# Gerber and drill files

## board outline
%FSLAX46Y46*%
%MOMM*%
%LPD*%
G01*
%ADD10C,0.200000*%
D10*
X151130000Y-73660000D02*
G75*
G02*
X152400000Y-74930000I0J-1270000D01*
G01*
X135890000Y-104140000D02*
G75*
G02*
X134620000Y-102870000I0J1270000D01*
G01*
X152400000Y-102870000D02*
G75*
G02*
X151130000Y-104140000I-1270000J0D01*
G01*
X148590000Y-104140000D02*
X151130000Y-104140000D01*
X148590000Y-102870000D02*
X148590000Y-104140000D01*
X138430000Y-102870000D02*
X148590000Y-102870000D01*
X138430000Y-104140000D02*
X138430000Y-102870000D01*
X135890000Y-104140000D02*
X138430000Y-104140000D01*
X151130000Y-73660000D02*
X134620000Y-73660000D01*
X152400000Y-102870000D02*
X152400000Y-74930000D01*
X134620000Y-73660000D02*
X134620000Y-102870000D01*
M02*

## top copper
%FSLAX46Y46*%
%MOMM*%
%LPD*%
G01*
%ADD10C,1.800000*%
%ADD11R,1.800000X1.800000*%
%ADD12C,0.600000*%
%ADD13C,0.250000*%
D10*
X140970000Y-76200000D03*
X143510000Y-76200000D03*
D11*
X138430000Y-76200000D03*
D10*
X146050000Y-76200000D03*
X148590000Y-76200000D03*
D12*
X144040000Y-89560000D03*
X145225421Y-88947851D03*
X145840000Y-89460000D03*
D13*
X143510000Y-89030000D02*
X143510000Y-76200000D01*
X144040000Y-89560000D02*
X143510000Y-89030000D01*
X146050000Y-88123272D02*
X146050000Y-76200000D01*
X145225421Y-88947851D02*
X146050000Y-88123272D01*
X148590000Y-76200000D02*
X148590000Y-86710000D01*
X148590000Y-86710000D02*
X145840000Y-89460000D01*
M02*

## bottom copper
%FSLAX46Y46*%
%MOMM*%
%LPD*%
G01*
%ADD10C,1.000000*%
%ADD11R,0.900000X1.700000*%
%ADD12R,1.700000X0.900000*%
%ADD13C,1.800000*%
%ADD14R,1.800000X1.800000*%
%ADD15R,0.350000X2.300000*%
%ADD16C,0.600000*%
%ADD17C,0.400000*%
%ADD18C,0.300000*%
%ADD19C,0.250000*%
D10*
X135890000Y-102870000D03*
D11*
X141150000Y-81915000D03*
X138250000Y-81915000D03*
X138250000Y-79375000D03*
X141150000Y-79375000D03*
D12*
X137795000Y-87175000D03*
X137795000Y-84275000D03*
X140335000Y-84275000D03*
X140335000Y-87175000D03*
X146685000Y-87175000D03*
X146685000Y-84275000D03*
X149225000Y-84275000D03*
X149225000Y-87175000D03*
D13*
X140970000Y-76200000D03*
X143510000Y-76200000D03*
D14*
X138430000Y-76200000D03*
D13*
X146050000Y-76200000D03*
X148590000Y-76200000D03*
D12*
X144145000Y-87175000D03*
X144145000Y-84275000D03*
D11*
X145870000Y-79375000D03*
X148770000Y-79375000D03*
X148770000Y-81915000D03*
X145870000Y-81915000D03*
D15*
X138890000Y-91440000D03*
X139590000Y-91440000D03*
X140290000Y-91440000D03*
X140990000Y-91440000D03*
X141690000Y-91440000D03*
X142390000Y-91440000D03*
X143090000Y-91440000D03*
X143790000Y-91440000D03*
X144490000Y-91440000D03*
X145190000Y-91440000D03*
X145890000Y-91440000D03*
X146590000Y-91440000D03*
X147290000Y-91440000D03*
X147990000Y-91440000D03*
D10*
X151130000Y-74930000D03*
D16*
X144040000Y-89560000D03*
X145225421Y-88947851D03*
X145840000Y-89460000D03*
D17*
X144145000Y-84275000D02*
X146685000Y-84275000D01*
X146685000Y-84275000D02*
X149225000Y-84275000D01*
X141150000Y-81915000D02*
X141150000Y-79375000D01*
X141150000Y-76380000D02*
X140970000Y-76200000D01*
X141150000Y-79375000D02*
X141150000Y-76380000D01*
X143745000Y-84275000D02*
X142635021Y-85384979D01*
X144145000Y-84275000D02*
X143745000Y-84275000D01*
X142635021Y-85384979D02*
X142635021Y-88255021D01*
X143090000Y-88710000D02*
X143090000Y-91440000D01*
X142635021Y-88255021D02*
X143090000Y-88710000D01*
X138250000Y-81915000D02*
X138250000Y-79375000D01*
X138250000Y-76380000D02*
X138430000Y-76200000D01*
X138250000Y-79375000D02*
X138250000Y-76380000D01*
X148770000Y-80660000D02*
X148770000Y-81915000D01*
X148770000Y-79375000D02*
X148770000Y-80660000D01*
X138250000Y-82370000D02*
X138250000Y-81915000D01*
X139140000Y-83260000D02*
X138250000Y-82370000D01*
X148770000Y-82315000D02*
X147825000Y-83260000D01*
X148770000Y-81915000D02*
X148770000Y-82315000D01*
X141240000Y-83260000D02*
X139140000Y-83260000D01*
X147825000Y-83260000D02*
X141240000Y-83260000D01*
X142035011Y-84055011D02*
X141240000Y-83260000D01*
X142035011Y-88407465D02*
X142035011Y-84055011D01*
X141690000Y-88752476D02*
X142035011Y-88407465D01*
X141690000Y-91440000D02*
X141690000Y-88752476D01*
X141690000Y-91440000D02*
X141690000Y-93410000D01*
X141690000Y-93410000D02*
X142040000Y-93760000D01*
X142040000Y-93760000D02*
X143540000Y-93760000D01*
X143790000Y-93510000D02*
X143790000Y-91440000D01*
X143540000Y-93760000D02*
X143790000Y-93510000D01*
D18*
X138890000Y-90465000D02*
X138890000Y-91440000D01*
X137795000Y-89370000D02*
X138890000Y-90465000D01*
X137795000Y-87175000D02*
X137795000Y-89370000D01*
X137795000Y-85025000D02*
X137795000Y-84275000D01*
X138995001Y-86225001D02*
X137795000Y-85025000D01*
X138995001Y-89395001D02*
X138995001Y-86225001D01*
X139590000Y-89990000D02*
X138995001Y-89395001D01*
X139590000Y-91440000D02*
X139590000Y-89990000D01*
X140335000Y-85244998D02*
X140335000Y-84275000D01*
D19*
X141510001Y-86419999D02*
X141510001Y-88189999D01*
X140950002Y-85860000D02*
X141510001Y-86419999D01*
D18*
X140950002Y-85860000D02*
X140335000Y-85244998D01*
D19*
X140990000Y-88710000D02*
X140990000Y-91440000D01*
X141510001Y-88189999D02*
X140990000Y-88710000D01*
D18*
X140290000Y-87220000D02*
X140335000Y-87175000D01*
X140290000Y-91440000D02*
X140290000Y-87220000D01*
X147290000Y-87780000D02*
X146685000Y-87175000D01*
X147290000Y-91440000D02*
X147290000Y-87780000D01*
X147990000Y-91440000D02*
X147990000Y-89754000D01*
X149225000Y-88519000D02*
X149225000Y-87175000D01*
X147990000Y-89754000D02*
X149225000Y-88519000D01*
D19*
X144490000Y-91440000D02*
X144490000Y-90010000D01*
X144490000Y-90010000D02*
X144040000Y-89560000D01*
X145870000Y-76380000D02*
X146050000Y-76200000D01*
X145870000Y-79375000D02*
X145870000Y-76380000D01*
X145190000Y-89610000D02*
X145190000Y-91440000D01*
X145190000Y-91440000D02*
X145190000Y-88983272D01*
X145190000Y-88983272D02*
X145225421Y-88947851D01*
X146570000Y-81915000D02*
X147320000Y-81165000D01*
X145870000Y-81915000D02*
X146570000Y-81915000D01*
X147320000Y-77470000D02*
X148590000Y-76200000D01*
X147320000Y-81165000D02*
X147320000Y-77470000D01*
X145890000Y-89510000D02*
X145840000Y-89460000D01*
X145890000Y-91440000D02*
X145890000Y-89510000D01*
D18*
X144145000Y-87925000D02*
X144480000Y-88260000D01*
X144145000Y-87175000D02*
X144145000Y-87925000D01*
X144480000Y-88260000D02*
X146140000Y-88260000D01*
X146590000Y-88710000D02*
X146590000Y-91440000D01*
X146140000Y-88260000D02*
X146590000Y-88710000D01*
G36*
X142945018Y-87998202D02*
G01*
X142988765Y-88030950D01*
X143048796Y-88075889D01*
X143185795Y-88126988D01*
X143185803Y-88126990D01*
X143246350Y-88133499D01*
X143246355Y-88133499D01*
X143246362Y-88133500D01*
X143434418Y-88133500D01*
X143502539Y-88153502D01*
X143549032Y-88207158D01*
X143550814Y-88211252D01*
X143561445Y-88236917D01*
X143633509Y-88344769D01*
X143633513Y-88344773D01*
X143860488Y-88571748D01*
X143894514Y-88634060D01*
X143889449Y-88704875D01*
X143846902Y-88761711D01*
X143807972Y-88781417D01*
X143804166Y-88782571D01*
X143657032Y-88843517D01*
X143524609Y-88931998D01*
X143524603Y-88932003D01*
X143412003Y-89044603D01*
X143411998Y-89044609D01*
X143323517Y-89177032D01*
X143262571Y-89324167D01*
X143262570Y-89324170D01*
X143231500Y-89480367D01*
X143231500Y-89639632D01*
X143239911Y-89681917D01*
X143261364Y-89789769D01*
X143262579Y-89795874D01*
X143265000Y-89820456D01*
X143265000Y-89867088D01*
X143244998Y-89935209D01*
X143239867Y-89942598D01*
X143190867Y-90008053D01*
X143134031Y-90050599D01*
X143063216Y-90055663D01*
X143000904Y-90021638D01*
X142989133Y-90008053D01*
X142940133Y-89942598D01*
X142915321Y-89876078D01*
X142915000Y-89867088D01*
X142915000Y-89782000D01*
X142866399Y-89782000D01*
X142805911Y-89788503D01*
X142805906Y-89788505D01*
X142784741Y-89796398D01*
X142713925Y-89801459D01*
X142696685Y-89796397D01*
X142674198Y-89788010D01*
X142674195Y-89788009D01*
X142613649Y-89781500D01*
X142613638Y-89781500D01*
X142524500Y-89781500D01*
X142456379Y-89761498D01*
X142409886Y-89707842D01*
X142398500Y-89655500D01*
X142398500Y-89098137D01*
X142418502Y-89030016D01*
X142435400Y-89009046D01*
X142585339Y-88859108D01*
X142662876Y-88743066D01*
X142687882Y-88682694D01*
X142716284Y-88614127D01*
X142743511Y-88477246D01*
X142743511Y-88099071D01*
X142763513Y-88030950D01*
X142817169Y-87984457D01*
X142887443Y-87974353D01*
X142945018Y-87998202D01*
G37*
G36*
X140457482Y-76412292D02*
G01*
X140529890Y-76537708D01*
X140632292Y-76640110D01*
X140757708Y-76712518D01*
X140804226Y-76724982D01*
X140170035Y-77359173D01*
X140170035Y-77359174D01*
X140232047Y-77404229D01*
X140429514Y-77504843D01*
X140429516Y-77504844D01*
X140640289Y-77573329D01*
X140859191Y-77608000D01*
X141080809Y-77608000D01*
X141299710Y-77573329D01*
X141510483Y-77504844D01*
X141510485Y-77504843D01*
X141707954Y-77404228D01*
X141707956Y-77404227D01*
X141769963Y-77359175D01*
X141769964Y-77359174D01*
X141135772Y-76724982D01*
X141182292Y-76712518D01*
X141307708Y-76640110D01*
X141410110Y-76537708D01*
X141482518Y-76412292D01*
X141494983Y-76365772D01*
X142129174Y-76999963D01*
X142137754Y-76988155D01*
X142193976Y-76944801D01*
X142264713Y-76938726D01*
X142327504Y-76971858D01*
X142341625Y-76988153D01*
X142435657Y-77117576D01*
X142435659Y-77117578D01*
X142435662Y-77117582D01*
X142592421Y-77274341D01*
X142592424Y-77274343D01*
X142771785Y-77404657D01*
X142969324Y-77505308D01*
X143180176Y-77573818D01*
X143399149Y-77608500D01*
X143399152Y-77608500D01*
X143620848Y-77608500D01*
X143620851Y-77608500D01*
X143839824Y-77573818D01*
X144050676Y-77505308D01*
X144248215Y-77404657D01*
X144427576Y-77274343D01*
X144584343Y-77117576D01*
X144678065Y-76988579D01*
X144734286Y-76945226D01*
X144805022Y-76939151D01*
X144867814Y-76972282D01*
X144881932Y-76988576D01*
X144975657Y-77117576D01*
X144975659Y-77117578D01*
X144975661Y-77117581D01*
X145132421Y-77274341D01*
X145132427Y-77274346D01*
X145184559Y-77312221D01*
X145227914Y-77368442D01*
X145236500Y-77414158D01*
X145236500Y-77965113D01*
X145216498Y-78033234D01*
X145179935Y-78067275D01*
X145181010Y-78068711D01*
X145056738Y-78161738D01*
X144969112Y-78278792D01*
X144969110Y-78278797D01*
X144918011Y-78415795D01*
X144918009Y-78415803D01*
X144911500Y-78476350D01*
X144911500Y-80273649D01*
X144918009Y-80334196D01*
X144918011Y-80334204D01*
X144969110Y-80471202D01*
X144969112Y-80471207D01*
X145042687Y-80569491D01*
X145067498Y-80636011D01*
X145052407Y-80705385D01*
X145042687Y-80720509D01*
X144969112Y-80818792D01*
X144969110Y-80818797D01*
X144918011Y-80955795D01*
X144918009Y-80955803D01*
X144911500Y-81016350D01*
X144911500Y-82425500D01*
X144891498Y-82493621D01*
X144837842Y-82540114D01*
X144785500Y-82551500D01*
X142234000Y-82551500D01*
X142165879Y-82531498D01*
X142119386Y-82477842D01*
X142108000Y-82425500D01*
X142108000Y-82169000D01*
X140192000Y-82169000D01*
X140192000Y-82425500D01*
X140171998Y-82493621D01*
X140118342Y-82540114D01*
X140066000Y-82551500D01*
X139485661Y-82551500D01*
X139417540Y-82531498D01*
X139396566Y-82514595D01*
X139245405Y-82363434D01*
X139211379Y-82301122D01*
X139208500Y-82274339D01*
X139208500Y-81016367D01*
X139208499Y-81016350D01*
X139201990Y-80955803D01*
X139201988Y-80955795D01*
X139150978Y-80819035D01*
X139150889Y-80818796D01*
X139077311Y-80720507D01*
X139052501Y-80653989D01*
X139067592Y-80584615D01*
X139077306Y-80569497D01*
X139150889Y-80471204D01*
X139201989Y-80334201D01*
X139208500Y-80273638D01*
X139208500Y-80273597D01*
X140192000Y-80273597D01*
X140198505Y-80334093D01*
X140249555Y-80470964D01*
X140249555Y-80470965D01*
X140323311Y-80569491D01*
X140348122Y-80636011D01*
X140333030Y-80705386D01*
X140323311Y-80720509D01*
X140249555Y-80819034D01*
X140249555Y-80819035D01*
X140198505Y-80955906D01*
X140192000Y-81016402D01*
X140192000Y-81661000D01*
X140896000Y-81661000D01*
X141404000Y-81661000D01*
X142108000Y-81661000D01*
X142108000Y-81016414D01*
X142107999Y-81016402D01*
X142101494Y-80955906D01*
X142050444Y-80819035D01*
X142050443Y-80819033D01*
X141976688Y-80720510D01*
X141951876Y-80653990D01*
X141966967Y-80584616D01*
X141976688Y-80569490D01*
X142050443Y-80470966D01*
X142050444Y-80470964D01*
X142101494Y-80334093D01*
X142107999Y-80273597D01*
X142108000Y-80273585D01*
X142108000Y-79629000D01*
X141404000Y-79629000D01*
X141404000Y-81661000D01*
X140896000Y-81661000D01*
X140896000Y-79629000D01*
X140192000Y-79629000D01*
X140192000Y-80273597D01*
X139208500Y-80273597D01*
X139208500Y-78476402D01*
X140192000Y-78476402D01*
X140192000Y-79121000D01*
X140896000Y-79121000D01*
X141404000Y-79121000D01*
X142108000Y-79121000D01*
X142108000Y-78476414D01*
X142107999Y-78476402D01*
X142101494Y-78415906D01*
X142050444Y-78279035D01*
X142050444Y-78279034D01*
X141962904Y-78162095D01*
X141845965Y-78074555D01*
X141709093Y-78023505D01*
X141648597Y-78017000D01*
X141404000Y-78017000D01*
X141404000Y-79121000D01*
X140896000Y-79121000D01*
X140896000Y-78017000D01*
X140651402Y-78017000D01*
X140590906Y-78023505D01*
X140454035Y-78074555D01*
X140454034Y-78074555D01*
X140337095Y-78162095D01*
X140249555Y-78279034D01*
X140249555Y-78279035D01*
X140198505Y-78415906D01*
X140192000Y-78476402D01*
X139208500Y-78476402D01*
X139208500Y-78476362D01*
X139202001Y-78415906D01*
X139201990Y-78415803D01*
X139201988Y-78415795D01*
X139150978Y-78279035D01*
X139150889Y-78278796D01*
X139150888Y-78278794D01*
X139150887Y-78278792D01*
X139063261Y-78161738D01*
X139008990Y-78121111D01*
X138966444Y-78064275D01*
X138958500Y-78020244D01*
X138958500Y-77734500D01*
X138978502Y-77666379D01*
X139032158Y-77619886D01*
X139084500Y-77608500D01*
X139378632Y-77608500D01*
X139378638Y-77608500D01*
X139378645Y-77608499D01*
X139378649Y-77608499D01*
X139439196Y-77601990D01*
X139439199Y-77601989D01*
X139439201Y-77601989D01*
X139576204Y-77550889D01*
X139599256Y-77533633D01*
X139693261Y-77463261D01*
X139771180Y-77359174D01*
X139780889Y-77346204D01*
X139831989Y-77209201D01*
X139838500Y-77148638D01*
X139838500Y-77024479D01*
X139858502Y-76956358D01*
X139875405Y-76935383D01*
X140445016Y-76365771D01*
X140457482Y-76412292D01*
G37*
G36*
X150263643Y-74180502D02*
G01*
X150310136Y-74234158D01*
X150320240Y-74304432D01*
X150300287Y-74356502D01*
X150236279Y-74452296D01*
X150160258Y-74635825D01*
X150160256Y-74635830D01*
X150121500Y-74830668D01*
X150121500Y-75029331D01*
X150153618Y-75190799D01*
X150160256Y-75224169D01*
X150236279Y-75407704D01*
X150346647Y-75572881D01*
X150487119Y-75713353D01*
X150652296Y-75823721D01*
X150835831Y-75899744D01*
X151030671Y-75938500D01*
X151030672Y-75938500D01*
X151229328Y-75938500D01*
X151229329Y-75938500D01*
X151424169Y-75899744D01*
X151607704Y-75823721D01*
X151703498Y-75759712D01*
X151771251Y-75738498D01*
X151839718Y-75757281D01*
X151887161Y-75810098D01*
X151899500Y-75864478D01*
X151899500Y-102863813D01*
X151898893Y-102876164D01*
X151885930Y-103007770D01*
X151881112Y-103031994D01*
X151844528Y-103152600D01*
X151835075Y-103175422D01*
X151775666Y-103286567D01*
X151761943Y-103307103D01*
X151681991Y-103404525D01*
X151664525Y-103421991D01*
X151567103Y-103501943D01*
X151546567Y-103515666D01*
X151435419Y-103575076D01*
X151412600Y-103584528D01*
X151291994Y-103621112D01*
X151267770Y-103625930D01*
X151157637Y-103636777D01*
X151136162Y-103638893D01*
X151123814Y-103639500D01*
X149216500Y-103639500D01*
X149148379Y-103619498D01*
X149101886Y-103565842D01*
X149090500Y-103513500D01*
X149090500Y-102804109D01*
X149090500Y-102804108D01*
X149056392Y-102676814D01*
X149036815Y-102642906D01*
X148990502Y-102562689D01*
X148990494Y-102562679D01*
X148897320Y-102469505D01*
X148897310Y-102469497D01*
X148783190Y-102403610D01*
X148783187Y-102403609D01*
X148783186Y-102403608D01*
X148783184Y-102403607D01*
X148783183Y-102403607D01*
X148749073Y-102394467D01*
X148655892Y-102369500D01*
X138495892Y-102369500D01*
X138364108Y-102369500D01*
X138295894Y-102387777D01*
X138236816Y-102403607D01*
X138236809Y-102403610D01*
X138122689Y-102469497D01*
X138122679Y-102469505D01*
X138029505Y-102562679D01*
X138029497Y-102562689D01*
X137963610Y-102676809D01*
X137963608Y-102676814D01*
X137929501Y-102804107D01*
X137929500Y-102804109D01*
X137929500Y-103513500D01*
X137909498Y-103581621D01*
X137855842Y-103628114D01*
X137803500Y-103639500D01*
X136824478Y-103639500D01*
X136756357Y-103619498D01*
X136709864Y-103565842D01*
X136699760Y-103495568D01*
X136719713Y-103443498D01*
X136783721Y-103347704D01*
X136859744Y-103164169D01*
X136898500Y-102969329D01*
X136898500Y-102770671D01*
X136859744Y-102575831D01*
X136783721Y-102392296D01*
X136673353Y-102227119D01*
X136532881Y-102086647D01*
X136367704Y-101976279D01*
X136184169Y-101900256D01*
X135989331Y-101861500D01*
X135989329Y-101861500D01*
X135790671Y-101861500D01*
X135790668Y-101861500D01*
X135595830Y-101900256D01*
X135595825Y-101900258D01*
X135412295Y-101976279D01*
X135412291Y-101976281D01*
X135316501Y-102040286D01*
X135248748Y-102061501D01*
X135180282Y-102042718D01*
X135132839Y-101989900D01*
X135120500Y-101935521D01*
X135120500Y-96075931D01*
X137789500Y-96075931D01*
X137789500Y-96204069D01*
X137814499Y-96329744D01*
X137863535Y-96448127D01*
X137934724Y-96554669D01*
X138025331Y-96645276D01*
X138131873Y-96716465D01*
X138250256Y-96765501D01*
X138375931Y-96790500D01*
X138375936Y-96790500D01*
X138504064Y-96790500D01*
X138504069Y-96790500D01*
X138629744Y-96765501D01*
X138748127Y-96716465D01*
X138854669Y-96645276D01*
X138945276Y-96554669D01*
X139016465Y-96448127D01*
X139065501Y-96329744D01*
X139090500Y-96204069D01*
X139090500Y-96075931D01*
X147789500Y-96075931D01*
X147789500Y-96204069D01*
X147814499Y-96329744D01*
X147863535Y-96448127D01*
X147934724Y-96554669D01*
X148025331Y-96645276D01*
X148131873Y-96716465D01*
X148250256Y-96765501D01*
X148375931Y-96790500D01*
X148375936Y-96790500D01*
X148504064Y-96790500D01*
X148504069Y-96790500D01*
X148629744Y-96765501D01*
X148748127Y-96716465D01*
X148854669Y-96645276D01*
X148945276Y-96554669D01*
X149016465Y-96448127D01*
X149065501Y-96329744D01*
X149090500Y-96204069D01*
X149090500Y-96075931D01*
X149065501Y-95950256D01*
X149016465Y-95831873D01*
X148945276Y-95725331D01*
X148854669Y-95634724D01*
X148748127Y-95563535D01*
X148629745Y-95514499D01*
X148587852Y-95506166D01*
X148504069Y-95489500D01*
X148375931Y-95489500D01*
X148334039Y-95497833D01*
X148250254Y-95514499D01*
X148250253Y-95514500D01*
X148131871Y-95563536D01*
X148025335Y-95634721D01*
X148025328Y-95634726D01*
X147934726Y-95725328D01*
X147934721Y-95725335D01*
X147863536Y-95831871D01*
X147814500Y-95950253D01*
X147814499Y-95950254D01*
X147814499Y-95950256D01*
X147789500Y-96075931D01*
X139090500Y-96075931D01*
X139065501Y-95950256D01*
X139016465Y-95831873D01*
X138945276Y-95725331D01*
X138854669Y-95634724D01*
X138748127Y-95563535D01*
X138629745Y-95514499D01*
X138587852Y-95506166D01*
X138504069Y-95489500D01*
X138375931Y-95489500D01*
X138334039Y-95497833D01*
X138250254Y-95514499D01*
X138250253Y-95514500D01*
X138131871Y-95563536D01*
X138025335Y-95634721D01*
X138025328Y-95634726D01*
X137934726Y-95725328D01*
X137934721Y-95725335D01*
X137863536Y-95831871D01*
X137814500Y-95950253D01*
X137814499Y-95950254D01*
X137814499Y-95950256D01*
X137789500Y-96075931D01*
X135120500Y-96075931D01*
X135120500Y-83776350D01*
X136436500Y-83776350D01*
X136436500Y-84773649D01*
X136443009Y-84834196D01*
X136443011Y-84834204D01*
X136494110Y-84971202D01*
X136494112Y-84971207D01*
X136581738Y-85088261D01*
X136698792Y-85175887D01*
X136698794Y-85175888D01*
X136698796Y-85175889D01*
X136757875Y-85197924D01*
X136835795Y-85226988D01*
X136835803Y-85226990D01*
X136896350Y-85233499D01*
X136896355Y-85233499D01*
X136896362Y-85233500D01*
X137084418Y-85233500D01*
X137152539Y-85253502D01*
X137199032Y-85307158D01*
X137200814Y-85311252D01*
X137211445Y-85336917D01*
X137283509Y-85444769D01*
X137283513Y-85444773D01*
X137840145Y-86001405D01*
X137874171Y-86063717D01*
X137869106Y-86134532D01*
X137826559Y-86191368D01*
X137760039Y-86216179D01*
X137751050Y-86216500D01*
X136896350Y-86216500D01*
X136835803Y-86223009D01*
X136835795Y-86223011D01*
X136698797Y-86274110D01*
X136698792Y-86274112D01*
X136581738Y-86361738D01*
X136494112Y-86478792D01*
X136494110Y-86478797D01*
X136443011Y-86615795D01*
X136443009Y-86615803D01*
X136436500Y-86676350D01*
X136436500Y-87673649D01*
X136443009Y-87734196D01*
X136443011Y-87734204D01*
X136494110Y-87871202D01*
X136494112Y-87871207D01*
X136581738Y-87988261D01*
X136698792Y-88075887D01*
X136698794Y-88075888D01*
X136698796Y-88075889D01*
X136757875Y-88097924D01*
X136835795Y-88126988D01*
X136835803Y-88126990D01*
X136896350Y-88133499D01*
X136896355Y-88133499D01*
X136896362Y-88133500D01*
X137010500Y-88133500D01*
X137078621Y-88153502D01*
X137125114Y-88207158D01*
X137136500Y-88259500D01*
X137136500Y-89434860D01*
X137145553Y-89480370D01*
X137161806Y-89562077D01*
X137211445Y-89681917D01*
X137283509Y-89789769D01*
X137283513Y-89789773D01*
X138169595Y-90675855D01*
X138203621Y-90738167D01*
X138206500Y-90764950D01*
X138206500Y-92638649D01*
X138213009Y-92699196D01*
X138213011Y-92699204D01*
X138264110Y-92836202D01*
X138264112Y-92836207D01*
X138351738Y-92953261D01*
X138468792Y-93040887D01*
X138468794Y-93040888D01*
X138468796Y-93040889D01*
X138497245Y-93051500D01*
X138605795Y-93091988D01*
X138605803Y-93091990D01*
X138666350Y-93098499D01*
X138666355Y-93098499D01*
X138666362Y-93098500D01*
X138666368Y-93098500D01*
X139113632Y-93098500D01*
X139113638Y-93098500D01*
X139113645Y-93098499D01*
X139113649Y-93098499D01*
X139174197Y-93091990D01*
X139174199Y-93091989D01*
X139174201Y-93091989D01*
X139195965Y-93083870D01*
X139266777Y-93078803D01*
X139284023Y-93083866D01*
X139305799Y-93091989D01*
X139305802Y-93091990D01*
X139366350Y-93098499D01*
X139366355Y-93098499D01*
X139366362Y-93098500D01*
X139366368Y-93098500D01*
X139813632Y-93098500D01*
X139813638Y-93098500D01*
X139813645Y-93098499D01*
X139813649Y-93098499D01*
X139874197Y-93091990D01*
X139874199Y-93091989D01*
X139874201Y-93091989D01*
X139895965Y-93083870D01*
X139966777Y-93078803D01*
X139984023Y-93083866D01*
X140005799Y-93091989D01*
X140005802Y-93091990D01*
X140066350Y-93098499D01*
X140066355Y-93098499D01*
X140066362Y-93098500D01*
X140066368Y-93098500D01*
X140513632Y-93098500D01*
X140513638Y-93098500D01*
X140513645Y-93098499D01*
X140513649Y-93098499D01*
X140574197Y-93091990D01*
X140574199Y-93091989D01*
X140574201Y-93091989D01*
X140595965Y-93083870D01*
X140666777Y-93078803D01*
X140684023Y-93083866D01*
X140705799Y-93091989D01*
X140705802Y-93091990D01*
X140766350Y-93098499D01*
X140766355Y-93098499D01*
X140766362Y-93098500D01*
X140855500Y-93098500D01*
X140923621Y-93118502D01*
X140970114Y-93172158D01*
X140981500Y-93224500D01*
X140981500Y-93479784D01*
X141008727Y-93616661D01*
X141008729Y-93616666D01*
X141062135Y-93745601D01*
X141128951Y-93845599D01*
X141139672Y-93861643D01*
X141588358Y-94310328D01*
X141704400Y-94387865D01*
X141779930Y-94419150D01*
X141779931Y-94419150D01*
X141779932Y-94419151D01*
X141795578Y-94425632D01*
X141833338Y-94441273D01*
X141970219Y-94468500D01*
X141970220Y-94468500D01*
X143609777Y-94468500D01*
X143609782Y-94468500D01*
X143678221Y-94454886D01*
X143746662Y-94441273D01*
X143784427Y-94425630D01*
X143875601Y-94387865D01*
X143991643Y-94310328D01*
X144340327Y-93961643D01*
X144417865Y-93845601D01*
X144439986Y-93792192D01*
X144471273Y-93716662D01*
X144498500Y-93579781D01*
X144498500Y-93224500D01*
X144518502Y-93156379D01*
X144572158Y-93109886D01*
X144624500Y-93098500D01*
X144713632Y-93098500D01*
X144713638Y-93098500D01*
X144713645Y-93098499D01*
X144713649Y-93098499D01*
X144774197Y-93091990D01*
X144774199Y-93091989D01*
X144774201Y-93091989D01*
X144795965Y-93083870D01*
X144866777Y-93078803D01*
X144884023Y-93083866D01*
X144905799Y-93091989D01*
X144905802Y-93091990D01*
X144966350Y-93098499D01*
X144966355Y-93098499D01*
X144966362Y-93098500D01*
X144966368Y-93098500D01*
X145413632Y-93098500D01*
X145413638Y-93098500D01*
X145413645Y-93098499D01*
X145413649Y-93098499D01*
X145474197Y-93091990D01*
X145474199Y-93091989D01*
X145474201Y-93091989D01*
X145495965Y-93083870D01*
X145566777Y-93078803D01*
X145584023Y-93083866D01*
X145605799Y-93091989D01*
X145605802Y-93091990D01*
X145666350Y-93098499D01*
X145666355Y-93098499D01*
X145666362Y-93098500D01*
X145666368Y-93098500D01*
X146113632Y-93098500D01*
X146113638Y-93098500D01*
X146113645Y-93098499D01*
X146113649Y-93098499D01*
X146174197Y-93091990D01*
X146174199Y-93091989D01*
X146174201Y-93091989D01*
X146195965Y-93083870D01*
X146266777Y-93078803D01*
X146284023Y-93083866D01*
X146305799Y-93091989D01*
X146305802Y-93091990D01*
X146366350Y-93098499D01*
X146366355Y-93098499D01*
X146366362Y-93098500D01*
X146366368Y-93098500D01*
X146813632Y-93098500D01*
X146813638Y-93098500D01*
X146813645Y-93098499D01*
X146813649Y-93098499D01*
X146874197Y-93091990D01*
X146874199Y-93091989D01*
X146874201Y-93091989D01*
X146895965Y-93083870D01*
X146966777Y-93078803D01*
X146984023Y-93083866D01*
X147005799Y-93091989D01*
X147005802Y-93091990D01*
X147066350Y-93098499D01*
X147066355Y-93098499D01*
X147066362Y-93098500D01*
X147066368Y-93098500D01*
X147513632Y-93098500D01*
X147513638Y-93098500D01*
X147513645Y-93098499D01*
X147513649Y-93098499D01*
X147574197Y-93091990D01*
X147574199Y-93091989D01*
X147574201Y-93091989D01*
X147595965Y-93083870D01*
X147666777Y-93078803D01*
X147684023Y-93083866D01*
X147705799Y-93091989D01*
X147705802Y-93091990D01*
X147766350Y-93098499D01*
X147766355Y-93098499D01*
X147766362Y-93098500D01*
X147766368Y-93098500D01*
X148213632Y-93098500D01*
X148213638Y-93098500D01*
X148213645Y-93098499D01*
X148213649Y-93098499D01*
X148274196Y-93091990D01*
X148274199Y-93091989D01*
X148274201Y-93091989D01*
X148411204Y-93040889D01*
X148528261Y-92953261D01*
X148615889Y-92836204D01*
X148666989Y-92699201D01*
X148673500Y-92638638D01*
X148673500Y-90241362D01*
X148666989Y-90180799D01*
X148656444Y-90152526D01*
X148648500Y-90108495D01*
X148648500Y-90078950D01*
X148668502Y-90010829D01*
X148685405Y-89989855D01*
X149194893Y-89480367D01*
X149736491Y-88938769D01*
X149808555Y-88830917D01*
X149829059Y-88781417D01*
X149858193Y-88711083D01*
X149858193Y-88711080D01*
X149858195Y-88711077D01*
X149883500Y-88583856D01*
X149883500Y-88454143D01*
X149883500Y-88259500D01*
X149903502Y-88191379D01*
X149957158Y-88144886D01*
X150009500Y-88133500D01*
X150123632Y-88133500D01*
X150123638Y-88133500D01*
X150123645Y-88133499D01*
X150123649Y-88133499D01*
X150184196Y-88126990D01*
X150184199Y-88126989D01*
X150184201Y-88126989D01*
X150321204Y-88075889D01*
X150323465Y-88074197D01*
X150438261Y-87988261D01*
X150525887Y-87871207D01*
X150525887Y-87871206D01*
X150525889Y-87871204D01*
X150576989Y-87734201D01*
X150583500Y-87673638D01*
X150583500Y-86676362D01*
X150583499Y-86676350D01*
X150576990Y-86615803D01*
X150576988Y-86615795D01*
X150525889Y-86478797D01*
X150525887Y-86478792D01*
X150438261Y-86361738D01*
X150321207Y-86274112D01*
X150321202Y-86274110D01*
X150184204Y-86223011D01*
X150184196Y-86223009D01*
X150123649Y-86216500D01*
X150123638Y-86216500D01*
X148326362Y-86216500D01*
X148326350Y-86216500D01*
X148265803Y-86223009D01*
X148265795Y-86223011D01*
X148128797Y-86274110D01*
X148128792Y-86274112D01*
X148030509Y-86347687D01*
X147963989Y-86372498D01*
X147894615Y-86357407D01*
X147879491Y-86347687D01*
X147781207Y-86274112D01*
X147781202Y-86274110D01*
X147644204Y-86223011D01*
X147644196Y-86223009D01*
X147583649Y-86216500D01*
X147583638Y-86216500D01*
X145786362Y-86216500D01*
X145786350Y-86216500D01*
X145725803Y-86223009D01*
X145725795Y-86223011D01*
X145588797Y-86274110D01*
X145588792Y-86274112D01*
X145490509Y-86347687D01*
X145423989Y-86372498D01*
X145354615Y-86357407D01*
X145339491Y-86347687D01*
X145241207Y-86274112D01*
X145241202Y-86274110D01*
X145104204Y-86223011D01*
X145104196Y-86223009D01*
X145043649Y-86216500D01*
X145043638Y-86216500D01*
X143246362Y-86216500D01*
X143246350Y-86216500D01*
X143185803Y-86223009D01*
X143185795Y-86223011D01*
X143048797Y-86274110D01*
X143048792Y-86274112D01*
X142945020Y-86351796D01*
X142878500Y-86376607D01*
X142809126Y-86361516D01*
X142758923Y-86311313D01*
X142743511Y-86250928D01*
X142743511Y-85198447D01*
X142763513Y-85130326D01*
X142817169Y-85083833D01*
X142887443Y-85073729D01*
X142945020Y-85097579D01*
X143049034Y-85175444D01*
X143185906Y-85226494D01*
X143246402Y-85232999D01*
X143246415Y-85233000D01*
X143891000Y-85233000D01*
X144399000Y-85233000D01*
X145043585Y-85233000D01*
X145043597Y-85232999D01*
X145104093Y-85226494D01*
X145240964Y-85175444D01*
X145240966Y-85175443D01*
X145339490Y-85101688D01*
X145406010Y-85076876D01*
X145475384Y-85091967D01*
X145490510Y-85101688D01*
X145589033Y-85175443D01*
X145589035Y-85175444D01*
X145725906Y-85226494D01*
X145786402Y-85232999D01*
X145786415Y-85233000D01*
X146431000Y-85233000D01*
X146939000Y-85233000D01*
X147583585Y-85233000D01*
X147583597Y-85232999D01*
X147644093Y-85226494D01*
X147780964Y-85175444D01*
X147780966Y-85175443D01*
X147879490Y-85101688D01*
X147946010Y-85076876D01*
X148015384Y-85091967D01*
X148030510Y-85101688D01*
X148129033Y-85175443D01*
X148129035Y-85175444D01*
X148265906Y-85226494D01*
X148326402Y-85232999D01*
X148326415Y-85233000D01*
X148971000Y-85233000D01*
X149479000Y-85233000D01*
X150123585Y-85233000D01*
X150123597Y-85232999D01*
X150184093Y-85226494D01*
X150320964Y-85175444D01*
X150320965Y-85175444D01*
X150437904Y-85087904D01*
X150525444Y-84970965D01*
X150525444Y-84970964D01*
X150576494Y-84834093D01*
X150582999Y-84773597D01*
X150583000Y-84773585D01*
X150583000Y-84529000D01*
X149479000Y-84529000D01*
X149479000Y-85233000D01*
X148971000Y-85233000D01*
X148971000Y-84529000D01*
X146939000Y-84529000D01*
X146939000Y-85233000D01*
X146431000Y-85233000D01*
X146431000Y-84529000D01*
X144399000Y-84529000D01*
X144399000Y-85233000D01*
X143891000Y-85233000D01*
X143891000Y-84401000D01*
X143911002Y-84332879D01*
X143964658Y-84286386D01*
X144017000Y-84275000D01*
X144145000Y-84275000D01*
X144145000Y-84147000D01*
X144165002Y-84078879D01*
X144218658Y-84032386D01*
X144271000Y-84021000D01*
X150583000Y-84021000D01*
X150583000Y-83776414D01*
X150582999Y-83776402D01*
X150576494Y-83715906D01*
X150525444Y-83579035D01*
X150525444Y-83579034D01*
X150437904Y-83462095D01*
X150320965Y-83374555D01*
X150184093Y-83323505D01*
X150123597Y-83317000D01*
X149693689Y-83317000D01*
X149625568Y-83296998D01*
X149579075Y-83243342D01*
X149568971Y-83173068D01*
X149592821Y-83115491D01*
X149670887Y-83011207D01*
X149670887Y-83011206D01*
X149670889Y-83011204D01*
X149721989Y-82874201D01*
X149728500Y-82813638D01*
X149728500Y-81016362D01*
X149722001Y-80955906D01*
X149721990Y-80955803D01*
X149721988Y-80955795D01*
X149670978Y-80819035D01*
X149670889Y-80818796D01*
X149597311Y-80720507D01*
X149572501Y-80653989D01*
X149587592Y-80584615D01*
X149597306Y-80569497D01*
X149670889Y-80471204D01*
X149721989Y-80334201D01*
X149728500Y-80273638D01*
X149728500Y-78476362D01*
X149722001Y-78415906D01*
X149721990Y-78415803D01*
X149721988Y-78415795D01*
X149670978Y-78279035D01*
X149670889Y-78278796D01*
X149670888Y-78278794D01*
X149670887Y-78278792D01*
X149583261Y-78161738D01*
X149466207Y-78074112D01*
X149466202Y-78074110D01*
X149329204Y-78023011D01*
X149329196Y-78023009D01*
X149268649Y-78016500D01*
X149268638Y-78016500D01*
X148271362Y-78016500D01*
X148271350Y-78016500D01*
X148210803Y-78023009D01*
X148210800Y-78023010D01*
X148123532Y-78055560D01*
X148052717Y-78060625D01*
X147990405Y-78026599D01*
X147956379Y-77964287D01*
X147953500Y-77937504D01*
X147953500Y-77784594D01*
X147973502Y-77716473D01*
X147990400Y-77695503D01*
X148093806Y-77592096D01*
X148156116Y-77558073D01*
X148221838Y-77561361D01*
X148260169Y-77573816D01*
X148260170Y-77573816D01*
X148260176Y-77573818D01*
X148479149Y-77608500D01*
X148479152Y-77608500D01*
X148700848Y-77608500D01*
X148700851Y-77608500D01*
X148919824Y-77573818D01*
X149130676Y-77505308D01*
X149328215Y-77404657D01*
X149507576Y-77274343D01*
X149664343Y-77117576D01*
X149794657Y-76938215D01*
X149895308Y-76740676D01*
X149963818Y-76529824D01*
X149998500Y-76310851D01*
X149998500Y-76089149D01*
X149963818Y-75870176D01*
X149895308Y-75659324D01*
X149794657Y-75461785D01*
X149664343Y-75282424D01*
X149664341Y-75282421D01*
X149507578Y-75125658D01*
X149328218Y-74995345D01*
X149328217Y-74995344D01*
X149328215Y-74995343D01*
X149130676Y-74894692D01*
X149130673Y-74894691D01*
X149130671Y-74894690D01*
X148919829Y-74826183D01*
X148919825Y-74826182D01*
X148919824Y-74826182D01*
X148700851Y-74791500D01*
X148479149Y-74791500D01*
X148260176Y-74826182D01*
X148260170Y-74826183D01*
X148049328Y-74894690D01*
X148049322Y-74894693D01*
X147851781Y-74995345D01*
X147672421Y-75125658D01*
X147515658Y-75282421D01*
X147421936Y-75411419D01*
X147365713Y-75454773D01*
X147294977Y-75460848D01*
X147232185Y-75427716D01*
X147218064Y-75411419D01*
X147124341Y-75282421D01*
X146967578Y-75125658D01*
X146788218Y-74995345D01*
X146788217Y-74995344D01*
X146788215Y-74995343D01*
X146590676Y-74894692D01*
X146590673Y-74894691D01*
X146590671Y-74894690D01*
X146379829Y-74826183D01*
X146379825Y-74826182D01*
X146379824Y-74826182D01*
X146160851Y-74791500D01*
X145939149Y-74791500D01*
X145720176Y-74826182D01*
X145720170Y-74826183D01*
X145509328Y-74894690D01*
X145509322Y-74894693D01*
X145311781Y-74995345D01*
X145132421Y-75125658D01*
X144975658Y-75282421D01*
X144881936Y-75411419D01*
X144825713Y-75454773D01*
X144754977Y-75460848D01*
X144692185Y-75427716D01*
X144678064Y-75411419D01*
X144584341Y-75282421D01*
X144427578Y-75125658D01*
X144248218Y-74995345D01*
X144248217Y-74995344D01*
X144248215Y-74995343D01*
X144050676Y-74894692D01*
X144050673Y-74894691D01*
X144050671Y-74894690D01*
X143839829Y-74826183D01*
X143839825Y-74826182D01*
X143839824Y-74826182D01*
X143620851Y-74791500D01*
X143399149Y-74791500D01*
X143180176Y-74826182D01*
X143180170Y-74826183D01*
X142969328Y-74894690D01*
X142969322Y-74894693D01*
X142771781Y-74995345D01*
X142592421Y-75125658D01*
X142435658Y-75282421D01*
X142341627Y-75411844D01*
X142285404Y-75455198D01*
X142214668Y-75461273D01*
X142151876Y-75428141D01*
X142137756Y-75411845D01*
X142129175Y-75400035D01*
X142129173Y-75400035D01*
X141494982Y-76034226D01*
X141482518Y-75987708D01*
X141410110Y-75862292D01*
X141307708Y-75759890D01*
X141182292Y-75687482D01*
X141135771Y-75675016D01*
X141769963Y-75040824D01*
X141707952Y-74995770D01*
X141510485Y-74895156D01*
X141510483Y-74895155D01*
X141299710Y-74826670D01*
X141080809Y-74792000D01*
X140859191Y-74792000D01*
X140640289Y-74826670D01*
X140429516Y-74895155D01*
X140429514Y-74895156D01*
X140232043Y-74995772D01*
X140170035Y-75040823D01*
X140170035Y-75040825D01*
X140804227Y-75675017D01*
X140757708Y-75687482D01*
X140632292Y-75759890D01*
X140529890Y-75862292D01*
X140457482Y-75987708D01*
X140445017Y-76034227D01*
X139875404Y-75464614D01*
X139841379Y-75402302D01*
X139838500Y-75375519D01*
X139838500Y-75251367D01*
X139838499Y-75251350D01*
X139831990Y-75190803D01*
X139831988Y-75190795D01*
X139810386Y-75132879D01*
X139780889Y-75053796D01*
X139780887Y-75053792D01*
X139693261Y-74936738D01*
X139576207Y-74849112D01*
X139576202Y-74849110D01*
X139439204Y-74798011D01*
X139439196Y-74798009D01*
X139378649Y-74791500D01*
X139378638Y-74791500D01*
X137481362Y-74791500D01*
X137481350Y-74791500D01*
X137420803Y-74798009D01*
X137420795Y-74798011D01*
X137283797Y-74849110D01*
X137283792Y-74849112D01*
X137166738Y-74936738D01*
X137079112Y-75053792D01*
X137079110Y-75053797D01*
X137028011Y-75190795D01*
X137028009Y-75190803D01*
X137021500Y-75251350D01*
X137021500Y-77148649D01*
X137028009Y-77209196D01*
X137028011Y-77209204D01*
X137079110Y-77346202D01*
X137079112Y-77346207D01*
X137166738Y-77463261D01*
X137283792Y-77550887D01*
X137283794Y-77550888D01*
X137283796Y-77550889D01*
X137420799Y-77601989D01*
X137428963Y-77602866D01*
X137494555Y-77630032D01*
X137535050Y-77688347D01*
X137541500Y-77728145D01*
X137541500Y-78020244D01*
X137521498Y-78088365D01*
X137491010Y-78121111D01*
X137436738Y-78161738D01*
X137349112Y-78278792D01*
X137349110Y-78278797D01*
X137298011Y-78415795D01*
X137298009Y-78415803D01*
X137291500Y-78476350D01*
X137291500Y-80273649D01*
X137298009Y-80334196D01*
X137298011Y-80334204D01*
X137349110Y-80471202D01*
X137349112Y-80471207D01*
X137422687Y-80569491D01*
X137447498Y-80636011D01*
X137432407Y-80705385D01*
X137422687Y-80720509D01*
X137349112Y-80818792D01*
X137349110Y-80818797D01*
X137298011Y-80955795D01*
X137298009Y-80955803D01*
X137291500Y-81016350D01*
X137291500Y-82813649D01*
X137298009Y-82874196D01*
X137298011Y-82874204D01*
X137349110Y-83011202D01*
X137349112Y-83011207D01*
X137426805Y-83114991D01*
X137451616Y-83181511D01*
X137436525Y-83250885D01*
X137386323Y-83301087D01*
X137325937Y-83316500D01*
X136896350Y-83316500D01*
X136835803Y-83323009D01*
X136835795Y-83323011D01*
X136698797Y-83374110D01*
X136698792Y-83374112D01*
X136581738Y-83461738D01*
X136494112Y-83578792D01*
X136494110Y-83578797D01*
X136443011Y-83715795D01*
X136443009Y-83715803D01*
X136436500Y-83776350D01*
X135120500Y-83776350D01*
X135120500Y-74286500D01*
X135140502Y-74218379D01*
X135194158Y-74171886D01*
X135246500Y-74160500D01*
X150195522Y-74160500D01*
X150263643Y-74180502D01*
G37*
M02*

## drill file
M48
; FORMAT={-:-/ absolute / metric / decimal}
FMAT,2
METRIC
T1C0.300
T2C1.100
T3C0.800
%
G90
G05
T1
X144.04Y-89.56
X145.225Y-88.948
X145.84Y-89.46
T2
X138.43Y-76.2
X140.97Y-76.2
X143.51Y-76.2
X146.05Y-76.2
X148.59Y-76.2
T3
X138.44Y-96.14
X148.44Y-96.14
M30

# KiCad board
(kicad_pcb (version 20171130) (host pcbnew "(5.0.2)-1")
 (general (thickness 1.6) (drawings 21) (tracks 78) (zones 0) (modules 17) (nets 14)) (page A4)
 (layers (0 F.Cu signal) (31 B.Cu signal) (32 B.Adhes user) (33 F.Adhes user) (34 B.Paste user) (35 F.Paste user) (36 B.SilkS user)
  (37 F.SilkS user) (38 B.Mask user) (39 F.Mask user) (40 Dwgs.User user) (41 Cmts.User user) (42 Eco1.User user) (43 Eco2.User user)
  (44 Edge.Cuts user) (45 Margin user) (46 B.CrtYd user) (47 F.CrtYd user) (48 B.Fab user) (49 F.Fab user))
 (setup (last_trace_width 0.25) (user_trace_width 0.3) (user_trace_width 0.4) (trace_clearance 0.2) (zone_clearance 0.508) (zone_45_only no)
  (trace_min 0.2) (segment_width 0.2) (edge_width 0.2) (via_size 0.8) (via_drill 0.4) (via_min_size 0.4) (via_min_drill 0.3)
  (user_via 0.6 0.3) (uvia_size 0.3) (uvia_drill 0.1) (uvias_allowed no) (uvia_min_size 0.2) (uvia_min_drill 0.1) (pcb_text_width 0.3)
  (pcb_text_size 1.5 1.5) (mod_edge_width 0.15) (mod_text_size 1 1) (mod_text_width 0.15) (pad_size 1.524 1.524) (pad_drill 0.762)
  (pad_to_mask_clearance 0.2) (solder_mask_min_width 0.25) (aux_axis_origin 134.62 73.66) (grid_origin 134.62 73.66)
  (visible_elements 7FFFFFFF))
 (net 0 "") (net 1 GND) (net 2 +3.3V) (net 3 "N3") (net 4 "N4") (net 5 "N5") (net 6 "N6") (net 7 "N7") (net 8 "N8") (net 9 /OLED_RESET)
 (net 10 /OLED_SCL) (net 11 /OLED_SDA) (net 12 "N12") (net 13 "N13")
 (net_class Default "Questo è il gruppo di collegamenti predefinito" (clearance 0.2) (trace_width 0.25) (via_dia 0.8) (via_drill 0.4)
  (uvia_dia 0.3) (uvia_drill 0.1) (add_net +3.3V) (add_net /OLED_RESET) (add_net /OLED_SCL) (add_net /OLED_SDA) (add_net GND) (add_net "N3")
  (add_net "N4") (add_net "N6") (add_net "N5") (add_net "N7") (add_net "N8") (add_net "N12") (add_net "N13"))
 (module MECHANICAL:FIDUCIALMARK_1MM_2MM (layer B.Cu) (at 135.89 102.87)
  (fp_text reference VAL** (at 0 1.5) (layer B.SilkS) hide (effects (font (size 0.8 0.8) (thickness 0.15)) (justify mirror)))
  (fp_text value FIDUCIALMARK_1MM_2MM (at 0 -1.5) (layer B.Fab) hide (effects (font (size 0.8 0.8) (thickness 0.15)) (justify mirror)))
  (pad "" smd circle (at 0 0) (size 1 1) (layers B.Cu)) (pad 1 smd circle (at 0 0) (size 2 2) (layers B.Mask)))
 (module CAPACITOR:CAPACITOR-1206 (layer B.Cu) (at 139.7 81.915 180)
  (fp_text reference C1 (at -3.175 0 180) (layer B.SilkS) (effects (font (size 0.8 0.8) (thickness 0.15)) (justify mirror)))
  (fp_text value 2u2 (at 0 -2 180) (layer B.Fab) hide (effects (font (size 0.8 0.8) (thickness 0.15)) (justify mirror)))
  (pad 1 smd rect (at -1.45 0 180) (size 0.9 1.7) (layers B.Cu B.Paste B.Mask) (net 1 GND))
  (pad 2 smd rect (at 1.45 0 180) (size 0.9 1.7) (layers B.Cu B.Paste B.Mask) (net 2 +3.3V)))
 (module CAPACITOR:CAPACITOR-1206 (layer B.Cu) (at 139.7 79.375 180)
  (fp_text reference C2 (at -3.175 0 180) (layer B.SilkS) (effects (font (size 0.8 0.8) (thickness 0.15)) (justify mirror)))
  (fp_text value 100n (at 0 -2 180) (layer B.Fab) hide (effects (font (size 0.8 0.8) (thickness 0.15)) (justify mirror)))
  (pad 2 smd rect (at 1.45 0 180) (size 0.9 1.7) (layers B.Cu B.Paste B.Mask) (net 2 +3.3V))
  (pad 1 smd rect (at -1.45 0 180) (size 0.9 1.7) (layers B.Cu B.Paste B.Mask) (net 1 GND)))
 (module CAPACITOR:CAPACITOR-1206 (layer B.Cu) (at 137.795 85.725 90)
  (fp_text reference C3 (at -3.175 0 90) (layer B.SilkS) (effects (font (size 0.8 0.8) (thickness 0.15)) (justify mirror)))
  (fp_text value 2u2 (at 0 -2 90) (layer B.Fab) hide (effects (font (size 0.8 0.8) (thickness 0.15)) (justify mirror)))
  (pad 1 smd rect (at -1.45 0 90) (size 0.9 1.7) (layers B.Cu B.Paste B.Mask) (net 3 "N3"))
  (pad 2 smd rect (at 1.45 0 90) (size 0.9 1.7) (layers B.Cu B.Paste B.Mask) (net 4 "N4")))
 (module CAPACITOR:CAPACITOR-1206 (layer B.Cu) (at 140.335 85.725 90)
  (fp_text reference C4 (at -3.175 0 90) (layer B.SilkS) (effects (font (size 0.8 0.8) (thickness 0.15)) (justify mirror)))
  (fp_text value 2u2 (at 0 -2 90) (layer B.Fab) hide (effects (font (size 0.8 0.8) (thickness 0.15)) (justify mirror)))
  (pad 2 smd rect (at 1.45 0 90) (size 0.9 1.7) (layers B.Cu B.Paste B.Mask) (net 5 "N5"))
  (pad 1 smd rect (at -1.45 0 90) (size 0.9 1.7) (layers B.Cu B.Paste B.Mask) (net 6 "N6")))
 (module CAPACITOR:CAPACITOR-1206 (layer B.Cu) (at 146.685 85.725 270)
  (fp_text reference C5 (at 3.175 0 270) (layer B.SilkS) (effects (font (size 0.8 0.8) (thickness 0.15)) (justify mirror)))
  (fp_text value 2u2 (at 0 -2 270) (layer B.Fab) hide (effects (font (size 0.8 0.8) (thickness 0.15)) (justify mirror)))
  (pad 2 smd rect (at 1.45 0 270) (size 0.9 1.7) (layers B.Cu B.Paste B.Mask) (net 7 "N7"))
  (pad 1 smd rect (at -1.45 0 270) (size 0.9 1.7) (layers B.Cu B.Paste B.Mask) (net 1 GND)))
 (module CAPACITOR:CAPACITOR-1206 (layer B.Cu) (at 149.225 85.725 270)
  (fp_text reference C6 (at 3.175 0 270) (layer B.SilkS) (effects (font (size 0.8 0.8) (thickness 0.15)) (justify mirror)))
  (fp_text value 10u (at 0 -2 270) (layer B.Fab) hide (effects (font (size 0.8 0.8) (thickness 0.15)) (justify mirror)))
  (pad 1 smd rect (at -1.45 0 270) (size 0.9 1.7) (layers B.Cu B.Paste B.Mask) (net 1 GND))
  (pad 2 smd rect (at 1.45 0 270) (size 0.9 1.7) (layers B.Cu B.Paste B.Mask) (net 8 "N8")))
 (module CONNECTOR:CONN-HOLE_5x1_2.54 (layer F.Cu) (at 143.51 76.2)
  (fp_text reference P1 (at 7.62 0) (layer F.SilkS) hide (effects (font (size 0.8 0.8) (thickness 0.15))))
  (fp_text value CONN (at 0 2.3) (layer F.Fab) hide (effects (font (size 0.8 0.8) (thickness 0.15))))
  (pad 2 thru_hole circle (at -2.54 0) (size 1.8 1.8) (drill 1.1) (layers *.Cu *.Mask) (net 1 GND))
  (pad 3 thru_hole circle (at 0 0) (size 1.8 1.8) (drill 1.1) (layers *.Cu *.Mask) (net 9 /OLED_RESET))
  (pad 1 thru_hole rect (at -5.08 0) (size 1.8 1.8) (drill 1.1) (layers *.Cu *.Mask) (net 2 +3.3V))
  (pad 4 thru_hole circle (at 2.54 0) (size 1.8 1.8) (drill 1.1) (layers *.Cu *.Mask) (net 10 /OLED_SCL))
  (pad 5 thru_hole circle (at 5.08 0) (size 1.8 1.8) (drill 1.1) (layers *.Cu *.Mask) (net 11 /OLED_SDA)))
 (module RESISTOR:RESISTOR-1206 (layer B.Cu) (at 144.145 85.725 90)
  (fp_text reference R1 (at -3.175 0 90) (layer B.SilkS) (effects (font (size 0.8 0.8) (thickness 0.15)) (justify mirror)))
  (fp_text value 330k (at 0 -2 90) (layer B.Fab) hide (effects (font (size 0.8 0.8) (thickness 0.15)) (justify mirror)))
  (pad 1 smd rect (at -1.45 0 90) (size 0.9 1.7) (layers B.Cu B.Paste B.Mask) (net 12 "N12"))
  (pad 2 smd rect (at 1.45 0 90) (size 0.9 1.7) (layers B.Cu B.Paste B.Mask) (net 1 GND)))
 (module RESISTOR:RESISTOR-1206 (layer B.Cu) (at 147.32 79.375 180)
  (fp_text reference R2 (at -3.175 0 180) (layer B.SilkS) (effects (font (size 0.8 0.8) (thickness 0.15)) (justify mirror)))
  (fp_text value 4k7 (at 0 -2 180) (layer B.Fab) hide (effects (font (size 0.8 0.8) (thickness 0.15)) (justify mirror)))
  (pad 2 smd rect (at 1.45 0 180) (size 0.9 1.7) (layers B.Cu B.Paste B.Mask) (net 10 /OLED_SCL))
  (pad 1 smd rect (at -1.45 0 180) (size 0.9 1.7) (layers B.Cu B.Paste B.Mask) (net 2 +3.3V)))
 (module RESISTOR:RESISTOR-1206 (layer B.Cu) (at 147.32 81.915 180)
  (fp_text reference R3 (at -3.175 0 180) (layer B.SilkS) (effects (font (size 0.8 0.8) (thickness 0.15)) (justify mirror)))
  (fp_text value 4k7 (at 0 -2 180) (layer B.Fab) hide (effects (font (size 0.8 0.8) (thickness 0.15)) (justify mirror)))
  (pad 1 smd rect (at -1.45 0 180) (size 0.9 1.7) (layers B.Cu B.Paste B.Mask) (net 2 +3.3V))
  (pad 2 smd rect (at 1.45 0 180) (size 0.9 1.7) (layers B.Cu B.Paste B.Mask) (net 11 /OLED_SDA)))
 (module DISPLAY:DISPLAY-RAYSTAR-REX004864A (layer B.Cu) (at 143.44 91.44)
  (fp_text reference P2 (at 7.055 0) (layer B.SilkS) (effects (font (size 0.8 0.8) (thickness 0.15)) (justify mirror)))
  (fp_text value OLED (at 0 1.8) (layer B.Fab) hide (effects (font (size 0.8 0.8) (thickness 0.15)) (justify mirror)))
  (pad 1 smd rect (at -4.55 0) (size 0.35 2.3) (layers B.Cu B.Paste B.Mask) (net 3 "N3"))
  (pad 2 smd rect (at -3.85 0) (size 0.35 2.3) (layers B.Cu B.Paste B.Mask) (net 4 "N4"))
  (pad 3 smd rect (at -3.15 0) (size 0.35 2.3) (layers B.Cu B.Paste B.Mask) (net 6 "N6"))
  (pad 4 smd rect (at -2.45 0) (size 0.35 2.3) (layers B.Cu B.Paste B.Mask) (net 5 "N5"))
  (pad 5 smd rect (at -1.75 0) (size 0.35 2.3) (layers B.Cu B.Paste B.Mask) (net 2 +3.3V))
  (pad 6 smd rect (at -1.05 0) (size 0.35 2.3) (layers B.Cu B.Paste B.Mask) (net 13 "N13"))
  (pad 7 smd rect (at -0.35 0) (size 0.35 2.3) (layers B.Cu B.Paste B.Mask) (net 1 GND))
  (pad 8 smd rect (at 0.35 0) (size 0.35 2.3) (layers B.Cu B.Paste B.Mask) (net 2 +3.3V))
  (pad 9 smd rect (at 1.05 0) (size 0.35 2.3) (layers B.Cu B.Paste B.Mask) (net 9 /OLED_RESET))
  (pad 10 smd rect (at 1.75 0) (size 0.35 2.3) (layers B.Cu B.Paste B.Mask) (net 10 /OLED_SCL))
  (pad 11 smd rect (at 2.45 0) (size 0.35 2.3) (layers B.Cu B.Paste B.Mask) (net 11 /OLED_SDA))
  (pad 12 smd rect (at 3.15 0) (size 0.35 2.3) (layers B.Cu B.Paste B.Mask) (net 12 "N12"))
  (pad 13 smd rect (at 3.85 0) (size 0.35 2.3) (layers B.Cu B.Paste B.Mask) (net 7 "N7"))
  (pad 14 smd rect (at 4.55 0) (size 0.35 2.3) (layers B.Cu B.Paste B.Mask) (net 8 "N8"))
  (pad "" np_thru_hole circle (at -5 4.7) (size 0.8 0.8) (drill 0.8) (layers *.Cu *.Mask))
  (pad "" np_thru_hole circle (at 5 4.7) (size 0.8 0.8) (drill 0.8) (layers *.Cu *.Mask)))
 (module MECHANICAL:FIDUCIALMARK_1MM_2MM (layer B.Cu) (at 151.13 74.93)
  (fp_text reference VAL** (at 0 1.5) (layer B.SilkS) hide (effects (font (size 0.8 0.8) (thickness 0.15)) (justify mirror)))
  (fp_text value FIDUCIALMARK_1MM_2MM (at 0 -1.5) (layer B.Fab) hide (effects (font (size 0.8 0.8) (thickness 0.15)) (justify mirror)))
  (pad 1 smd circle (at 0 0) (size 2 2) (layers B.Mask)) (pad "" smd circle (at 0 0) (size 1 1) (layers B.Cu)))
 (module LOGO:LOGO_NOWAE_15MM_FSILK (layer B.Cu) (at 143.42 99.66 180)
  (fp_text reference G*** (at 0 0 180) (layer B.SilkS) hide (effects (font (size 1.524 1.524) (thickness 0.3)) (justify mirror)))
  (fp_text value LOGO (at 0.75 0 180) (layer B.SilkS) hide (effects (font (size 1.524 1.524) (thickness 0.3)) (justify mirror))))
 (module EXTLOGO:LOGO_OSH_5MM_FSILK (layer B.Cu) (at 143.62 95.66 180)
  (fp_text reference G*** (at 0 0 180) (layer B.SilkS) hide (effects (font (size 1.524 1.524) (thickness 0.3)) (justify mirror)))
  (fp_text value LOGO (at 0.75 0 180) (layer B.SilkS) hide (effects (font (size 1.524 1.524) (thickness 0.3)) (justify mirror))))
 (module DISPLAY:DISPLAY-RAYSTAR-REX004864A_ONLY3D (layer F.Cu) (at 143.52 90.06)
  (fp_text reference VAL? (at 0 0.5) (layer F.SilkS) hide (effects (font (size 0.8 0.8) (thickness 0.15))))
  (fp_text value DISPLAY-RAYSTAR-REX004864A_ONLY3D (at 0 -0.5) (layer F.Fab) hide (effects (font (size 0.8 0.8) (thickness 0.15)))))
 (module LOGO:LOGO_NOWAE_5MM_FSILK (layer F.Cu) (at 143.42 102.06)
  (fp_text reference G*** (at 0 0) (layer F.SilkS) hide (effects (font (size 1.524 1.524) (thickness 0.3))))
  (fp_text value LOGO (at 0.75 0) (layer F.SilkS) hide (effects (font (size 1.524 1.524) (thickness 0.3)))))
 (gr_arc (start 151.13 74.93) (end 152.4 74.93) (angle -90) (layer Edge.Cuts) (width 0.2))
 (gr_arc (start 135.89 102.87) (end 134.62 102.87) (angle -90) (layer Edge.Cuts) (width 0.2))
 (gr_arc (start 151.13 102.87) (end 151.13 104.14) (angle -90) (layer Edge.Cuts) (width 0.2))
 (gr_line (start 148.59 104.14) (end 151.13 104.14) (layer Edge.Cuts) (width 0.2))
 (gr_line (start 148.59 102.87) (end 148.59 104.14) (layer Edge.Cuts) (width 0.2))
 (gr_line (start 138.43 102.87) (end 148.59 102.87) (layer Edge.Cuts) (width 0.2))
 (gr_line (start 138.43 104.14) (end 138.43 102.87) (layer Edge.Cuts) (width 0.2))
 (gr_line (start 135.89 104.14) (end 138.43 104.14) (layer Edge.Cuts) (width 0.2))
 (gr_line (start 151.13 73.66) (end 134.62 73.66) (layer Edge.Cuts) (width 0.2))
 (gr_line (start 152.4 102.87) (end 152.4 74.93) (layer Edge.Cuts) (width 0.2))
 (gr_line (start 134.62 73.66) (end 134.62 102.87) (layer Edge.Cuts) (width 0.2))
 (segment (start 144.145 84.275) (end 146.685 84.275) (width 0.4) (layer B.Cu) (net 1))
 (segment (start 146.685 84.275) (end 149.225 84.275) (width 0.4) (layer B.Cu) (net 1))
 (segment (start 141.15 81.915) (end 141.15 79.375) (width 0.4) (layer B.Cu) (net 1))
 (segment (start 141.15 76.38) (end 140.97 76.2) (width 0.4) (layer B.Cu) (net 1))
 (segment (start 141.15 79.375) (end 141.15 76.38) (width 0.4) (layer B.Cu) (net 1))
 (segment (start 143.745 84.275) (end 142.635021 85.384979) (width 0.4) (layer B.Cu) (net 1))
 (segment (start 144.145 84.275) (end 143.745 84.275) (width 0.4) (layer B.Cu) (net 1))
 (segment (start 142.635021 85.384979) (end 142.635021 88.255021) (width 0.4) (layer B.Cu) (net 1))
 (segment (start 143.09 88.71) (end 143.09 91.44) (width 0.4) (layer B.Cu) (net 1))
 (segment (start 142.635021 88.255021) (end 143.09 88.71) (width 0.4) (layer B.Cu) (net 1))
 (segment (start 138.25 81.915) (end 138.25 79.375) (width 0.4) (layer B.Cu) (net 2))
 (segment (start 138.25 76.38) (end 138.43 76.2) (width 0.4) (layer B.Cu) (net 2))
 (segment (start 138.25 79.375) (end 138.25 76.38) (width 0.4) (layer B.Cu) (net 2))
 (segment (start 148.77 80.66) (end 148.77 81.915) (width 0.4) (layer B.Cu) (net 2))
 (segment (start 148.77 79.375) (end 148.77 80.66) (width 0.4) (layer B.Cu) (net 2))
 (segment (start 138.25 82.37) (end 138.25 81.915) (width 0.4) (layer B.Cu) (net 2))
 (segment (start 139.14 83.26) (end 138.25 82.37) (width 0.4) (layer B.Cu) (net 2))
 (segment (start 148.77 82.315) (end 147.825 83.26) (width 0.4) (layer B.Cu) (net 2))
 (segment (start 148.77 81.915) (end 148.77 82.315) (width 0.4) (layer B.Cu) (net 2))
 (segment (start 141.24 83.26) (end 139.14 83.26) (width 0.4) (layer B.Cu) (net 2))
 (segment (start 147.825 83.26) (end 141.24 83.26) (width 0.4) (layer B.Cu) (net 2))
 (segment (start 142.035011 84.055011) (end 141.24 83.26) (width 0.4) (layer B.Cu) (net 2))
 (segment (start 142.035011 88.407465) (end 142.035011 84.055011) (width 0.4) (layer B.Cu) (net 2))
 (segment (start 141.69 88.752476) (end 142.035011 88.407465) (width 0.4) (layer B.Cu) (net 2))
 (segment (start 141.69 91.44) (end 141.69 88.752476) (width 0.4) (layer B.Cu) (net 2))
 (segment (start 141.69 91.44) (end 141.69 93.41) (width 0.4) (layer B.Cu) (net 2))
 (segment (start 141.69 93.41) (end 142.04 93.76) (width 0.4) (layer B.Cu) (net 2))
 (segment (start 142.04 93.76) (end 143.54 93.76) (width 0.4) (layer B.Cu) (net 2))
 (segment (start 143.79 93.51) (end 143.79 91.44) (width 0.4) (layer B.Cu) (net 2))
 (segment (start 143.54 93.76) (end 143.79 93.51) (width 0.4) (layer B.Cu) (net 2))
 (segment (start 138.89 90.465) (end 138.89 91.44) (width 0.3) (layer B.Cu) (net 3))
 (segment (start 137.795 89.37) (end 138.89 90.465) (width 0.3) (layer B.Cu) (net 3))
 (segment (start 137.795 87.175) (end 137.795 89.37) (width 0.3) (layer B.Cu) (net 3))
 (segment (start 137.795 85.025) (end 137.795 84.275) (width 0.3) (layer B.Cu) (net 4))
 (segment (start 138.995001 86.225001) (end 137.795 85.025) (width 0.3) (layer B.Cu) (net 4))
 (segment (start 138.995001 89.395001) (end 138.995001 86.225001) (width 0.3) (layer B.Cu) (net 4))
 (segment (start 139.59 89.99) (end 138.995001 89.395001) (width 0.3) (layer B.Cu) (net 4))
 (segment (start 139.59 91.44) (end 139.59 89.99) (width 0.3) (layer B.Cu) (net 4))
 (segment (start 140.335 85.244998) (end 140.335 84.275) (width 0.3) (layer B.Cu) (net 5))
 (segment (start 141.510001 86.419999) (end 141.510001 88.189999) (width 0.25) (layer B.Cu) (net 5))
 (segment (start 140.950002 85.86) (end 141.510001 86.419999) (width 0.25) (layer B.Cu) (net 5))
 (segment (start 140.950002 85.86) (end 140.335 85.244998) (width 0.3) (layer B.Cu) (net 5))
 (segment (start 140.99 88.71) (end 140.99 91.44) (width 0.25) (layer B.Cu) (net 5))
 (segment (start 141.510001 88.189999) (end 140.99 88.71) (width 0.25) (layer B.Cu) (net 5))
 (segment (start 140.29 87.22) (end 140.335 87.175) (width 0.3) (layer B.Cu) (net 6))
 (segment (start 140.29 91.44) (end 140.29 87.22) (width 0.3) (layer B.Cu) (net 6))
 (segment (start 147.29 87.78) (end 146.685 87.175) (width 0.3) (layer B.Cu) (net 7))
 (segment (start 147.29 91.44) (end 147.29 87.78) (width 0.3) (layer B.Cu) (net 7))
 (segment (start 147.99 91.44) (end 147.99 89.754) (width 0.3) (layer B.Cu) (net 8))
 (segment (start 149.225 88.519) (end 149.225 87.175) (width 0.3) (layer B.Cu) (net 8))
 (segment (start 147.99 89.754) (end 149.225 88.519) (width 0.3) (layer B.Cu) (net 8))
 (via (at 144.04 89.56) (size 0.6) (drill 0.3) (layers F.Cu B.Cu) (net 9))
 (segment (start 144.49 91.44) (end 144.49 90.01) (width 0.25) (layer B.Cu) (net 9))
 (segment (start 144.49 90.01) (end 144.04 89.56) (width 0.25) (layer B.Cu) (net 9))
 (segment (start 143.51 89.03) (end 143.51 76.2) (width 0.25) (layer F.Cu) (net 9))
 (segment (start 144.04 89.56) (end 143.51 89.03) (width 0.25) (layer F.Cu) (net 9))
 (segment (start 145.87 76.38) (end 146.05 76.2) (width 0.25) (layer B.Cu) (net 10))
 (segment (start 145.87 79.375) (end 145.87 76.38) (width 0.25) (layer B.Cu) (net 10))
 (segment (start 145.19 89.61) (end 145.19 91.44) (width 0.25) (layer B.Cu) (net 10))
 (via (at 145.225421 88.947851) (size 0.6) (drill 0.3) (layers F.Cu B.Cu) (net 10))
 (segment (start 145.19 91.44) (end 145.19 88.983272) (width 0.25) (layer B.Cu) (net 10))
 (segment (start 145.19 88.983272) (end 145.225421 88.947851) (width 0.25) (layer B.Cu) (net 10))
 (segment (start 146.05 88.123272) (end 146.05 76.2) (width 0.25) (layer F.Cu) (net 10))
 (segment (start 145.225421 88.947851) (end 146.05 88.123272) (width 0.25) (layer F.Cu) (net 10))
 (segment (start 146.57 81.915) (end 147.32 81.165) (width 0.25) (layer B.Cu) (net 11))
 (segment (start 145.87 81.915) (end 146.57 81.915) (width 0.25) (layer B.Cu) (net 11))
 (segment (start 147.32 77.47) (end 148.59 76.2) (width 0.25) (layer B.Cu) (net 11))
 (segment (start 147.32 81.165) (end 147.32 77.47) (width 0.25) (layer B.Cu) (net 11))
 (via (at 145.84 89.46) (size 0.6) (drill 0.3) (layers F.Cu B.Cu) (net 11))
 (segment (start 148.59 76.2) (end 148.59 86.71) (width 0.25) (layer F.Cu) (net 11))
 (segment (start 148.59 86.71) (end 145.84 89.46) (width 0.25) (layer F.Cu) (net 11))
 (segment (start 145.89 89.51) (end 145.84 89.46) (width 0.25) (layer B.Cu) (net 11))
 (segment (start 145.89 91.44) (end 145.89 89.51) (width 0.25) (layer B.Cu) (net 11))
 (segment (start 144.145 87.925) (end 144.48 88.26) (width 0.3) (layer B.Cu) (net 12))
 (segment (start 144.145 87.175) (end 144.145 87.925) (width 0.3) (layer B.Cu) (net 12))
 (segment (start 144.48 88.26) (end 146.14 88.26) (width 0.3) (layer B.Cu) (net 12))
 (segment (start 146.59 88.71) (end 146.59 91.44) (width 0.3) (layer B.Cu) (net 12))
 (segment (start 146.14 88.26) (end 146.59 88.71) (width 0.3) (layer B.Cu) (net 12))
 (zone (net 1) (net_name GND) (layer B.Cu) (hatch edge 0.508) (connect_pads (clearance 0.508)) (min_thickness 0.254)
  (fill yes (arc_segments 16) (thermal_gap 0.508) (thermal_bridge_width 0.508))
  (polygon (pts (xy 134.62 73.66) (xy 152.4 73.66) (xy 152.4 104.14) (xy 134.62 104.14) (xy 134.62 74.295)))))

